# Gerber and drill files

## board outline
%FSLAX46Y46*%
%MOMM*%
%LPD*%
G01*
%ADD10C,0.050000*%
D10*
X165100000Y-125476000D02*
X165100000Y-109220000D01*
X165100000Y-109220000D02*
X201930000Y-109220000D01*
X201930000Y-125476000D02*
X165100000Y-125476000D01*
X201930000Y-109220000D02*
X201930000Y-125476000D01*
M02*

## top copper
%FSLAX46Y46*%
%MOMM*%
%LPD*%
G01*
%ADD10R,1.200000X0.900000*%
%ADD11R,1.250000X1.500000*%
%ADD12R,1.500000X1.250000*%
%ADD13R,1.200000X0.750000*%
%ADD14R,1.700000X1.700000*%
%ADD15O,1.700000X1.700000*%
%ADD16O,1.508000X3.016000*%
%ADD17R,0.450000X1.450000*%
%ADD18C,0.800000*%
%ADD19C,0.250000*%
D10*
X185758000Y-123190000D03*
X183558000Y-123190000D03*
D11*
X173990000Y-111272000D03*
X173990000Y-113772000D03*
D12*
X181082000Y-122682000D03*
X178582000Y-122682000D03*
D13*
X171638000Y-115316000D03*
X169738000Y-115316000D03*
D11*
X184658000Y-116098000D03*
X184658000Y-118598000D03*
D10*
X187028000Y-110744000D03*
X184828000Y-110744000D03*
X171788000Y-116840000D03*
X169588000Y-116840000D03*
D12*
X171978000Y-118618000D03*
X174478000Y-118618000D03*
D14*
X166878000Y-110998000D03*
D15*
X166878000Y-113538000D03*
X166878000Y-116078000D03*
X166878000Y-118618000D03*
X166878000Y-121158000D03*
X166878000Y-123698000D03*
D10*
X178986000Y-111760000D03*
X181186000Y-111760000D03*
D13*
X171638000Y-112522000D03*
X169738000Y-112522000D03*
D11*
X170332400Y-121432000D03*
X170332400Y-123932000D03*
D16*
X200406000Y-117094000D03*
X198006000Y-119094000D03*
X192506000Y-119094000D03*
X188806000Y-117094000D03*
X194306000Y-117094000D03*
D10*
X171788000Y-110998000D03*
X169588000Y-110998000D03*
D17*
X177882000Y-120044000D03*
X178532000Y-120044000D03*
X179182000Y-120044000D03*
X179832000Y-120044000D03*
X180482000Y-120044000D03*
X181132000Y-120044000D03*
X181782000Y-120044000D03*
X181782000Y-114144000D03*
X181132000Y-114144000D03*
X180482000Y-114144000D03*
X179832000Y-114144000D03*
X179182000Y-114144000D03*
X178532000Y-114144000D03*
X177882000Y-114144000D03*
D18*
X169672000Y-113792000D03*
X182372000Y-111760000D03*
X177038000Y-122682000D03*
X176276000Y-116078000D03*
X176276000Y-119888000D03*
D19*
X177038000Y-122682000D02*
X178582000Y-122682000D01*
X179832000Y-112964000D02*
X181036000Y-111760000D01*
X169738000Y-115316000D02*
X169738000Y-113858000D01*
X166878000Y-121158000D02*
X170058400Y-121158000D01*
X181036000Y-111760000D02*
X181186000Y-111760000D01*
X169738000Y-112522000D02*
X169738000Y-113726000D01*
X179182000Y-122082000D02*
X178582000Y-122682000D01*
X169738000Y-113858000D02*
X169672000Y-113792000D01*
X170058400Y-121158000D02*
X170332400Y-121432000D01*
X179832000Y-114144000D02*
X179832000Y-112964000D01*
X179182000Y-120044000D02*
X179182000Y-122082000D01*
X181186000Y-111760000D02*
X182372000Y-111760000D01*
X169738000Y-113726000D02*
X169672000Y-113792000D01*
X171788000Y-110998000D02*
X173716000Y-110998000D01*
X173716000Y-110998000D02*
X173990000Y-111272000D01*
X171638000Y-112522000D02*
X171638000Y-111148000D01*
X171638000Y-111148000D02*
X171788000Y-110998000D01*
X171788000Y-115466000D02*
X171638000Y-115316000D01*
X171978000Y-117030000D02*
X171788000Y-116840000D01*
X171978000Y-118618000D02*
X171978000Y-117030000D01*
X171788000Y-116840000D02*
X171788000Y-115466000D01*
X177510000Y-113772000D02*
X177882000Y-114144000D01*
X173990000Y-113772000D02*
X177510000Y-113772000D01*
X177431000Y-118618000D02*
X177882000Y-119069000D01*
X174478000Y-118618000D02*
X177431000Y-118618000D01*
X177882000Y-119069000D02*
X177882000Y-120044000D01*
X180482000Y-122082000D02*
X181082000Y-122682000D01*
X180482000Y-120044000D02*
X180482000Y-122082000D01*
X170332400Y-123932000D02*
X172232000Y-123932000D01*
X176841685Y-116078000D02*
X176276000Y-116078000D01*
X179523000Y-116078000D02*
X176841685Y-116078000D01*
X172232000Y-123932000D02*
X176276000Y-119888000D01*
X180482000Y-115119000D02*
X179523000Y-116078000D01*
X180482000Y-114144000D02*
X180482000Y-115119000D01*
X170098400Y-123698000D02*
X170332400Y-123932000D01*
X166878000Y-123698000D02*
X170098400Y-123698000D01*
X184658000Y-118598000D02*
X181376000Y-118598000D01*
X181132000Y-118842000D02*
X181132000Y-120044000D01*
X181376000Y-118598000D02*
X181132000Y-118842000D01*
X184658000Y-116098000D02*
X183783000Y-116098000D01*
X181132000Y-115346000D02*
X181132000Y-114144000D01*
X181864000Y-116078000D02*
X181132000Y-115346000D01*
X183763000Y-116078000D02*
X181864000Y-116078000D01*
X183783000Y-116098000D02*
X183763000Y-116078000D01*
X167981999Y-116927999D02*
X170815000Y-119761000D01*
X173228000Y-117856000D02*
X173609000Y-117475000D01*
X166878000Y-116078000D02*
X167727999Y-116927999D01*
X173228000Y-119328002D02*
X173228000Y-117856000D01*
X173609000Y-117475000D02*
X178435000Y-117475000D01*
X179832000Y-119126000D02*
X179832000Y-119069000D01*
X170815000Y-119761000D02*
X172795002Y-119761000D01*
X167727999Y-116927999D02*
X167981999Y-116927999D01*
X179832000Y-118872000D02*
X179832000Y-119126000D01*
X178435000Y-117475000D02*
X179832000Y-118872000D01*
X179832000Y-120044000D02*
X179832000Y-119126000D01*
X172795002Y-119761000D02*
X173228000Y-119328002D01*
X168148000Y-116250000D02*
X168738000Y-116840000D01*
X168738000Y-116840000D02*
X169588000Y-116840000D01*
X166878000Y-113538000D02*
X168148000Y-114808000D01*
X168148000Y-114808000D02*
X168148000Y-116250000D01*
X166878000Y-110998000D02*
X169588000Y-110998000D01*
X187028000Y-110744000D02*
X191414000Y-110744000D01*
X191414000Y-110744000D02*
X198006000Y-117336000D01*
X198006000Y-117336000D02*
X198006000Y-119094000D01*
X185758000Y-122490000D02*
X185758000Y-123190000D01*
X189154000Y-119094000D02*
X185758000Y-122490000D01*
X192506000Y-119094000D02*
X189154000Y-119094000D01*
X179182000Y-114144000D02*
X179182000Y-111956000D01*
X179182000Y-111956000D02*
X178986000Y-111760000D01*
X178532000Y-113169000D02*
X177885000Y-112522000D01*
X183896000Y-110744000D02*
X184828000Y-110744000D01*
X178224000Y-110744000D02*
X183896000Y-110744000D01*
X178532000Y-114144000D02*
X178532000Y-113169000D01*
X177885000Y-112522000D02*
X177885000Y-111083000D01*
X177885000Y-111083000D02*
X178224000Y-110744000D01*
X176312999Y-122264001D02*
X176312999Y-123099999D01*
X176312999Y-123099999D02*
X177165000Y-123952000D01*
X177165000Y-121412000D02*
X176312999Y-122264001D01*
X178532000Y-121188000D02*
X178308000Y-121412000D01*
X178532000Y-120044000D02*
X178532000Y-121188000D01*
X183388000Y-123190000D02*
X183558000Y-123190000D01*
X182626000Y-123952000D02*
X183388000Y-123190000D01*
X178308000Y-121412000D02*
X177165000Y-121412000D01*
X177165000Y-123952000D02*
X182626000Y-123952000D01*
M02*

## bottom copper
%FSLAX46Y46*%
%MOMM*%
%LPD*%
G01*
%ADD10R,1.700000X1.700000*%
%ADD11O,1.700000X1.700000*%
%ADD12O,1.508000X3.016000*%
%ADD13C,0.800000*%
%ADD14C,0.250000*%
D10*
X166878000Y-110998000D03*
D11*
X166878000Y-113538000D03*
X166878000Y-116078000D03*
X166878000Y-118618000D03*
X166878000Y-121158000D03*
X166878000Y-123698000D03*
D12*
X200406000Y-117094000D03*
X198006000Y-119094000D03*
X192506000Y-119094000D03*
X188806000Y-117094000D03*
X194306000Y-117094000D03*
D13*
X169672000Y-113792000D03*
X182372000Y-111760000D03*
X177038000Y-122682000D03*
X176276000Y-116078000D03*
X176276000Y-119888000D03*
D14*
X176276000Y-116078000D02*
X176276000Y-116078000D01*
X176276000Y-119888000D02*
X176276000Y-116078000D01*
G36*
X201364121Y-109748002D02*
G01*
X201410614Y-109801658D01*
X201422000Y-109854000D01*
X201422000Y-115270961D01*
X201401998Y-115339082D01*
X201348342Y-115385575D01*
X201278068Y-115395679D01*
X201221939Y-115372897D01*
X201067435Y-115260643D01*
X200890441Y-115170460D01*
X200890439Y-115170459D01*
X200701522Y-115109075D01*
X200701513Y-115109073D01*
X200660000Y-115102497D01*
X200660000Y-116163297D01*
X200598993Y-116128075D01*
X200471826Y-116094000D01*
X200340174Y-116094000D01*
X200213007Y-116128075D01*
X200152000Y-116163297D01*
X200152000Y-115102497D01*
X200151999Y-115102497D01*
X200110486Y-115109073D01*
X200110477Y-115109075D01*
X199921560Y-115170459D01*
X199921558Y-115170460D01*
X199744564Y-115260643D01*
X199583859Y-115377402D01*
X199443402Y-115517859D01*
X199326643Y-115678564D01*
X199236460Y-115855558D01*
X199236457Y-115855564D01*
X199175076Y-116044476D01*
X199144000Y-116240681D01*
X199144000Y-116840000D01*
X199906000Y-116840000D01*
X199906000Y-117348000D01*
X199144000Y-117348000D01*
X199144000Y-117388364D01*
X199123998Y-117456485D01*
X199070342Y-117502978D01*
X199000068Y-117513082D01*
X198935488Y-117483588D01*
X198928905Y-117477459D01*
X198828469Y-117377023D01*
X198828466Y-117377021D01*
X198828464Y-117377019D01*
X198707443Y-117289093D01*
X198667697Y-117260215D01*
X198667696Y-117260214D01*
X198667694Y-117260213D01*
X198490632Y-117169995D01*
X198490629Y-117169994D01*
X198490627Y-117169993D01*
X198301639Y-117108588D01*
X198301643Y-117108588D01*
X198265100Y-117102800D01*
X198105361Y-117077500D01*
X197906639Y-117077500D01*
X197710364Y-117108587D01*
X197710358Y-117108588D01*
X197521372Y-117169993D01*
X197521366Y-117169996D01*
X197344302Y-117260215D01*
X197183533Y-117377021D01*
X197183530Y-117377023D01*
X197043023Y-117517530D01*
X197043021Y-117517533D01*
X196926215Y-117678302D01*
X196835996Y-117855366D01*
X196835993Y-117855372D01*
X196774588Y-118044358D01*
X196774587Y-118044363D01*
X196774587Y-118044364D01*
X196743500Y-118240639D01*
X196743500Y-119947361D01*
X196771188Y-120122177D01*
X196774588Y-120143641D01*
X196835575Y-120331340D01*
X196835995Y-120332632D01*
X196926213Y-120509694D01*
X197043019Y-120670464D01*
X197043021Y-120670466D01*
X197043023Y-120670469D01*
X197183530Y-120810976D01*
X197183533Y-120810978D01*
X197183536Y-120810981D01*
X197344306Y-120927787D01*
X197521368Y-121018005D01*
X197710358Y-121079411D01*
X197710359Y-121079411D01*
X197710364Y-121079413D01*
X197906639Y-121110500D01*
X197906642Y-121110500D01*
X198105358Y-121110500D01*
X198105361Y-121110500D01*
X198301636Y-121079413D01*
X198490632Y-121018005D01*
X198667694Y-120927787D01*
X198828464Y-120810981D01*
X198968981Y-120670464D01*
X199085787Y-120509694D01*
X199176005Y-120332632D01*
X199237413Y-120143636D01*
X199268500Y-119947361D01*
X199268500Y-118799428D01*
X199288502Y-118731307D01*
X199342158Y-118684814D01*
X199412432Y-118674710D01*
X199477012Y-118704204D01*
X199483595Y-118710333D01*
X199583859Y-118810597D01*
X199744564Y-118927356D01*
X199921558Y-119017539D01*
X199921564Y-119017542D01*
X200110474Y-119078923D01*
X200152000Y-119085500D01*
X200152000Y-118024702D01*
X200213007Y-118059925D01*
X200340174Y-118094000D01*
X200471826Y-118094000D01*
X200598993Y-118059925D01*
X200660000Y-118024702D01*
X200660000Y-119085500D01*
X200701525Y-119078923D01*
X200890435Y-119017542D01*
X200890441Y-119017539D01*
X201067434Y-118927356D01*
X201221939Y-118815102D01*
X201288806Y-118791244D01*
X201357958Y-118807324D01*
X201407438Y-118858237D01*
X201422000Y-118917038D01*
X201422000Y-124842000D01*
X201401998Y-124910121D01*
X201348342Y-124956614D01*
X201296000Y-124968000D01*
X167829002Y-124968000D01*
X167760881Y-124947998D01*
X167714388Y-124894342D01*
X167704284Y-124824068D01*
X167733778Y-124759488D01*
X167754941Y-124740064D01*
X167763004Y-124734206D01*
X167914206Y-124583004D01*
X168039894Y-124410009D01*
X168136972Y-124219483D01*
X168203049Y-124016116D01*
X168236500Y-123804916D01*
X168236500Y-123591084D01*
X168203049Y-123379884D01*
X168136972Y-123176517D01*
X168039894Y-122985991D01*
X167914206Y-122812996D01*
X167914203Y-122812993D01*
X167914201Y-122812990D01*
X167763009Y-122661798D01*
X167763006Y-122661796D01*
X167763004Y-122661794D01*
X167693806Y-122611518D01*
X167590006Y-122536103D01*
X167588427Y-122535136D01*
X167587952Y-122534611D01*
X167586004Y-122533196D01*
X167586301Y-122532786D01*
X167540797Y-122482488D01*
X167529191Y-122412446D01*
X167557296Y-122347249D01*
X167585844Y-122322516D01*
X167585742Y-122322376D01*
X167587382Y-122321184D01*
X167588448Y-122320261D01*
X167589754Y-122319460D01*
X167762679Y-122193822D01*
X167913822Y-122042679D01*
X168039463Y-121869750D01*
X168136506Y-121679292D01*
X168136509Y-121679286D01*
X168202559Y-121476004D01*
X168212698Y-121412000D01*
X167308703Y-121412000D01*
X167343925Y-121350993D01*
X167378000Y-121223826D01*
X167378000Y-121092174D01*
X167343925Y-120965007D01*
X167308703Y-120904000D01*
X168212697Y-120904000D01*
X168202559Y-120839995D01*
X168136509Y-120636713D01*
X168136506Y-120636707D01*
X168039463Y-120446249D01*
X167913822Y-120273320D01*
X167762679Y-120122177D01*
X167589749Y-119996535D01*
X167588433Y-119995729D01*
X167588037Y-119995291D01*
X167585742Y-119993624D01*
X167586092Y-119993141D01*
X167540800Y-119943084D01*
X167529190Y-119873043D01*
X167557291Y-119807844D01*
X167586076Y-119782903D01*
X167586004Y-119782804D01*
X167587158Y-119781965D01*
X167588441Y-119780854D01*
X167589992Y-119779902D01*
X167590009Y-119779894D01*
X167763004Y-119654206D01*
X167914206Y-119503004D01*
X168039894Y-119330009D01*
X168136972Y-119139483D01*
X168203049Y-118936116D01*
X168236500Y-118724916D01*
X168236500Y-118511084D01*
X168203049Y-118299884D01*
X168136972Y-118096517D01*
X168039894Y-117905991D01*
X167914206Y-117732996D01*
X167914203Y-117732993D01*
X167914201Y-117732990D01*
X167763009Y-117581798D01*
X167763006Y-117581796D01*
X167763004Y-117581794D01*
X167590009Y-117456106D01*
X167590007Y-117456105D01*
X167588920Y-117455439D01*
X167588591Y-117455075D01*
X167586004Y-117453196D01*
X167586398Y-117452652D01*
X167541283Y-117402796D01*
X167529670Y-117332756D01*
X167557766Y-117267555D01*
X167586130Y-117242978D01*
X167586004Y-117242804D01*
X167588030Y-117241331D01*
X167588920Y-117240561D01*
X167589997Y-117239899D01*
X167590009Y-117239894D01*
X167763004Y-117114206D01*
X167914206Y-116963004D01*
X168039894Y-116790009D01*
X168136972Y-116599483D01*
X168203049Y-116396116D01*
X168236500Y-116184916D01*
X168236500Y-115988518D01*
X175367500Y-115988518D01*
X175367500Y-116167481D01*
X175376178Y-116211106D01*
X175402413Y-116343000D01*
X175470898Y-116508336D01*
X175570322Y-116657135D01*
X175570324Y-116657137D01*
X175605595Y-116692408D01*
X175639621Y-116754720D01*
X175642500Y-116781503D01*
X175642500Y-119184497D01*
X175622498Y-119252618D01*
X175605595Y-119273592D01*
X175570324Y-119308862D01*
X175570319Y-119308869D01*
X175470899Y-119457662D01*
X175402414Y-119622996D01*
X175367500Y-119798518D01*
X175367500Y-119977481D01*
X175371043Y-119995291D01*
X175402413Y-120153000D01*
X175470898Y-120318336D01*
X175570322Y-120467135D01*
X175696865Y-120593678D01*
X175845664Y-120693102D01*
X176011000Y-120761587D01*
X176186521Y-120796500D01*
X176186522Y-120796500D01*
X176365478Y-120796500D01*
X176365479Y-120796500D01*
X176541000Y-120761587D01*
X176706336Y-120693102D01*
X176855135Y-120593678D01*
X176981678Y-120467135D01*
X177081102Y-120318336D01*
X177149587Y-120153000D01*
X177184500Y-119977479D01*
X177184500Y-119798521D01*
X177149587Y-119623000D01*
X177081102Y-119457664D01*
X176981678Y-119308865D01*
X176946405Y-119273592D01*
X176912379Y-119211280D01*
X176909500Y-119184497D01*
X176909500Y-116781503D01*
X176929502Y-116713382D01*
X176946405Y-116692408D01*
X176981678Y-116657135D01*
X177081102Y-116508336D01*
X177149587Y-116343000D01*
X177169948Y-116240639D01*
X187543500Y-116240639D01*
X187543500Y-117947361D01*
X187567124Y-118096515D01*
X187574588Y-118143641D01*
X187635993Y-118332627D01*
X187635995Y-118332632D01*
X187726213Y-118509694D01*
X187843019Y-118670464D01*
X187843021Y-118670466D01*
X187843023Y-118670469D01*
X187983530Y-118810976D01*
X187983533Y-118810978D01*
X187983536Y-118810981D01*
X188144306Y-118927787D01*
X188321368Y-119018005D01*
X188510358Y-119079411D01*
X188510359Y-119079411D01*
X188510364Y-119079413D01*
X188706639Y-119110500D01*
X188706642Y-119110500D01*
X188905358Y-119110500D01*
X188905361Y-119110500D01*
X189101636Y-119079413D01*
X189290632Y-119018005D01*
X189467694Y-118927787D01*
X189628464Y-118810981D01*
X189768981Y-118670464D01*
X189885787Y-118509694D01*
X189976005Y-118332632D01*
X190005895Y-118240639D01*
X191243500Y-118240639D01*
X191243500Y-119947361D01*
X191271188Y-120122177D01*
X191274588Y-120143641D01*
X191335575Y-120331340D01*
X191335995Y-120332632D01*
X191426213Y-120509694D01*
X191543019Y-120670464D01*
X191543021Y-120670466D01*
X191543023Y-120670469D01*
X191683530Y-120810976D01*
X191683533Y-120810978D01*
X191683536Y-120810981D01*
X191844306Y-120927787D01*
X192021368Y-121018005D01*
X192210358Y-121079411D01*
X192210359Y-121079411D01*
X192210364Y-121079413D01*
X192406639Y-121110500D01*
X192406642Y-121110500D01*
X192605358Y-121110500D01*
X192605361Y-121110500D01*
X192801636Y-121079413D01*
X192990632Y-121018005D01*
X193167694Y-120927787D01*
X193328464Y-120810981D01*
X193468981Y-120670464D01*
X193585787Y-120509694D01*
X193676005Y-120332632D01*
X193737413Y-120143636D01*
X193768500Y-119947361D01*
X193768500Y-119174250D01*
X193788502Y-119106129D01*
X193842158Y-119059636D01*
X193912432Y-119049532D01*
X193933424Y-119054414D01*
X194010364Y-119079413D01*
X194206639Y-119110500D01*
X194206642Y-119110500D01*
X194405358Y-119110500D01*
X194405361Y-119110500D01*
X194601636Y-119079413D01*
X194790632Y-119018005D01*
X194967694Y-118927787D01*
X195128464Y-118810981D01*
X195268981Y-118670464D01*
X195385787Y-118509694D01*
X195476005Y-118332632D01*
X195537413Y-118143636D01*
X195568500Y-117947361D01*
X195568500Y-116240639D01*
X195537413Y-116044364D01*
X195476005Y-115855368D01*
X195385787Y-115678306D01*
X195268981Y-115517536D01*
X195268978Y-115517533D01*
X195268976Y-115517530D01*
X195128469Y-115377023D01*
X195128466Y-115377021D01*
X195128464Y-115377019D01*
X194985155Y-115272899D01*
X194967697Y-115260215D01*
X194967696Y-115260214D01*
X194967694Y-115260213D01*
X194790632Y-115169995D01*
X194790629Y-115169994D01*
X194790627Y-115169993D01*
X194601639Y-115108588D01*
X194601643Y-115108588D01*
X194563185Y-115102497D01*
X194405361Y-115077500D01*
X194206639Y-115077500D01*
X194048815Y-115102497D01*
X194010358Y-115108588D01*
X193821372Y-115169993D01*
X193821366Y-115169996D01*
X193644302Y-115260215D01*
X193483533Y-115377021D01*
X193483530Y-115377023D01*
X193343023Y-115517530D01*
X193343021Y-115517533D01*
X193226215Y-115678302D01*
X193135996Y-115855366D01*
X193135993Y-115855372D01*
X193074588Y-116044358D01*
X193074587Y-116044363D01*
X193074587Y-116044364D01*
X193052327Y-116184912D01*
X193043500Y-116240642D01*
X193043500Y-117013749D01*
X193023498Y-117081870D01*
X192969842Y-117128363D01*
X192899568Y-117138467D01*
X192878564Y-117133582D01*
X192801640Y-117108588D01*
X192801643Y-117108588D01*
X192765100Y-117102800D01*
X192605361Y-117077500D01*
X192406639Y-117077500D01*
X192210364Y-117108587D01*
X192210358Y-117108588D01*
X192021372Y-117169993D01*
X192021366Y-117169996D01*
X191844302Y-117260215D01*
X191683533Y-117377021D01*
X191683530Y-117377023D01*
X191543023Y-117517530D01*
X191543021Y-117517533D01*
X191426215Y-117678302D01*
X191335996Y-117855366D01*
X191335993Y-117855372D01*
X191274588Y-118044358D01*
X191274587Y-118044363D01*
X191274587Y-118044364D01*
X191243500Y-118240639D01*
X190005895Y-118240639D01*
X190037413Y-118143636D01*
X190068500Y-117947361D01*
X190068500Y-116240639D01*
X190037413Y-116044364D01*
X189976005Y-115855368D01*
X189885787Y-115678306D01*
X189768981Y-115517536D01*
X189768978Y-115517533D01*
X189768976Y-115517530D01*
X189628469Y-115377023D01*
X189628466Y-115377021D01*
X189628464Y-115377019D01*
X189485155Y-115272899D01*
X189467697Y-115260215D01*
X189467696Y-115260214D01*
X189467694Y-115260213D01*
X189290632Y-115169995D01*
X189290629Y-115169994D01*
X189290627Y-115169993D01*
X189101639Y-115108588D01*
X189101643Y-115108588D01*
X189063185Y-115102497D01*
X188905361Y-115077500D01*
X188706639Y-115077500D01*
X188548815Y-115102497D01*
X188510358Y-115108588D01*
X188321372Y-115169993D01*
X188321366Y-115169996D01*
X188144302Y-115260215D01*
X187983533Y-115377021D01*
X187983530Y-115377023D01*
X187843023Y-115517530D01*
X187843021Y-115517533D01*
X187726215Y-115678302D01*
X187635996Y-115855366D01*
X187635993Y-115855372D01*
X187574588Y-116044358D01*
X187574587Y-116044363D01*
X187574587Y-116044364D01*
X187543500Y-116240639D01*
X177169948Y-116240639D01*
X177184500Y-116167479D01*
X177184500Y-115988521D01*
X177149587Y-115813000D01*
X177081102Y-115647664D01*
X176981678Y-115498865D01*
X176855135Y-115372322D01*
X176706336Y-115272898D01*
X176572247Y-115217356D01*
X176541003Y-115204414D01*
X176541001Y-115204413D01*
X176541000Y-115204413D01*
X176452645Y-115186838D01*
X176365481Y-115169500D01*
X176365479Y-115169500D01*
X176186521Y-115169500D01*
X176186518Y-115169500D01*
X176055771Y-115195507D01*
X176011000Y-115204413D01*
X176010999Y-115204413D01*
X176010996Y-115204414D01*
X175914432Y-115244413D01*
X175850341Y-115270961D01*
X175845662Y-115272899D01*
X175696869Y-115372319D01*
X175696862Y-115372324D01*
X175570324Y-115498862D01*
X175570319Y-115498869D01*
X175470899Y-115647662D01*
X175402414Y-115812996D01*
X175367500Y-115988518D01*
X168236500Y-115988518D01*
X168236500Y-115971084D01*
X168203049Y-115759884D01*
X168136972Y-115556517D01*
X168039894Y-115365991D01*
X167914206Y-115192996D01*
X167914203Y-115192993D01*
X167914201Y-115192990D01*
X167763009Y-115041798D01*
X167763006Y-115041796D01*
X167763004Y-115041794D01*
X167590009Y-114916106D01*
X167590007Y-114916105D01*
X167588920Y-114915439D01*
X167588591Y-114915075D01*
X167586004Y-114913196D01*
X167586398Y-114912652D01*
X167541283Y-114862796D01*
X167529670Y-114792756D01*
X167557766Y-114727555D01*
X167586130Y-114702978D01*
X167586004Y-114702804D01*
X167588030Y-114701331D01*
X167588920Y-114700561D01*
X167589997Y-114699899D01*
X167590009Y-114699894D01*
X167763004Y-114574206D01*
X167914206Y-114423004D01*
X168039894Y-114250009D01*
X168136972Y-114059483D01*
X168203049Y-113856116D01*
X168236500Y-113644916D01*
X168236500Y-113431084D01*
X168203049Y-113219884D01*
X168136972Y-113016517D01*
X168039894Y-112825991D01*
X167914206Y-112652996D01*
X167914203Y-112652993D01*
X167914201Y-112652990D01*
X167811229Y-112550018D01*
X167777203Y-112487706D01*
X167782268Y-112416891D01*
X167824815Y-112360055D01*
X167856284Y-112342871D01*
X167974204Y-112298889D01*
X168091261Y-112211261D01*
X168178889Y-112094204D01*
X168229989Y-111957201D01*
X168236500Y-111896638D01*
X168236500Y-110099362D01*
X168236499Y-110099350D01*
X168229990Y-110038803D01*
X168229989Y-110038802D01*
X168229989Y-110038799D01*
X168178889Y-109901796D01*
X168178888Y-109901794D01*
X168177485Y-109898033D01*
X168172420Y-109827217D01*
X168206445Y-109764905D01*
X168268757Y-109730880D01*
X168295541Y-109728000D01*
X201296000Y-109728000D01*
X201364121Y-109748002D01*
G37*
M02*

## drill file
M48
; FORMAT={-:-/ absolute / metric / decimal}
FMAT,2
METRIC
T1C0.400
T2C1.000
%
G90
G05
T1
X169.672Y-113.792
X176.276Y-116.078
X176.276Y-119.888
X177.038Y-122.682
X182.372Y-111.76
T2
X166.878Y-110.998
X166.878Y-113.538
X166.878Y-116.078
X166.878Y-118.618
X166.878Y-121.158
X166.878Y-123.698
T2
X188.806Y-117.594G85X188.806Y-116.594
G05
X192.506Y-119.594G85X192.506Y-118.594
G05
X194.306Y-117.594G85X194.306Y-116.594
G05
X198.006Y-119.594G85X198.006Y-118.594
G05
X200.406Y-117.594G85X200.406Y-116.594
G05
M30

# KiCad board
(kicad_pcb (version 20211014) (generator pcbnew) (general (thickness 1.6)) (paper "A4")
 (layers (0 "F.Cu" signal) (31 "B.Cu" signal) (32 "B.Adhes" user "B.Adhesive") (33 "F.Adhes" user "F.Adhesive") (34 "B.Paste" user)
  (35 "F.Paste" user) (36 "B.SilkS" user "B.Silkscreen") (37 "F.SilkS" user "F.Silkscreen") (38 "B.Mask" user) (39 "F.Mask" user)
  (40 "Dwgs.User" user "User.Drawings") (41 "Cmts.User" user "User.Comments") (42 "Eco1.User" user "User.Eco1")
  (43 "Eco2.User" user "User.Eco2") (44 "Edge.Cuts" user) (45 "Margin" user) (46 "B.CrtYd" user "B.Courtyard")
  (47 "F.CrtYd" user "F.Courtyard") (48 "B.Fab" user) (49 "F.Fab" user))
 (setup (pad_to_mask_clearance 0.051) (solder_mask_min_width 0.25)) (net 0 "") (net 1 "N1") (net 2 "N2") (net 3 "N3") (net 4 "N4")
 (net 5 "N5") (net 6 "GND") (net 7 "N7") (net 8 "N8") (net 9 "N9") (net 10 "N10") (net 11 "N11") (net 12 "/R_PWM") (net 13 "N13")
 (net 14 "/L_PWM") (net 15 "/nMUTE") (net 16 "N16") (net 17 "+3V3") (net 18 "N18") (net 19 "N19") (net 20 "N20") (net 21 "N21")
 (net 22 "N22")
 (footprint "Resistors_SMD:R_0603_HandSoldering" (layer "F.Cu") (at 184.658 123.19 180)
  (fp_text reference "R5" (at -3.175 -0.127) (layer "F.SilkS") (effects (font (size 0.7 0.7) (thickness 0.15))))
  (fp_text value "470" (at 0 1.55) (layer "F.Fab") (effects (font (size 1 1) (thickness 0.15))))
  (pad "1" smd rect locked (at -1.1 0 180) (size 1.2 0.9) (layers "F.Cu" "F.Paste" "F.Mask") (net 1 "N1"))
  (pad "2" smd rect locked (at 1.1 0 180) (size 1.2 0.9) (layers "F.Cu" "F.Paste" "F.Mask") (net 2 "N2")))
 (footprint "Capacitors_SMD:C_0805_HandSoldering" (layer "F.Cu") (at 173.99 112.522 -90)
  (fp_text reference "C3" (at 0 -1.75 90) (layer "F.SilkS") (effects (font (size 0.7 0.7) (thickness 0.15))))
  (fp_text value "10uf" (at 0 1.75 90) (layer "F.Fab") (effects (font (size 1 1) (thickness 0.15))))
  (pad "1" smd rect locked (at -1.25 0 270) (size 1.5 1.25) (layers "F.Cu" "F.Paste" "F.Mask") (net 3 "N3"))
  (pad "2" smd rect locked (at 1.25 0 270) (size 1.5 1.25) (layers "F.Cu" "F.Paste" "F.Mask") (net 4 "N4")))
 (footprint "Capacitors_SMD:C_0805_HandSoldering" (layer "F.Cu") (at 179.832 122.682 180)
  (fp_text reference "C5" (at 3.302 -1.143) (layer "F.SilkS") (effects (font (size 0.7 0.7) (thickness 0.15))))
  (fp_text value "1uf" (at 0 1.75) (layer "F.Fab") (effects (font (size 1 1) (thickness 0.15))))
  (pad "1" smd rect locked (at -1.25 0 180) (size 1.5 1.25) (layers "F.Cu" "F.Paste" "F.Mask") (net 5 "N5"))
  (pad "2" smd rect locked (at 1.25 0 180) (size 1.5 1.25) (layers "F.Cu" "F.Paste" "F.Mask") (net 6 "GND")))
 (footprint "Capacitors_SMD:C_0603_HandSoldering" (layer "F.Cu") (at 170.688 115.316 180)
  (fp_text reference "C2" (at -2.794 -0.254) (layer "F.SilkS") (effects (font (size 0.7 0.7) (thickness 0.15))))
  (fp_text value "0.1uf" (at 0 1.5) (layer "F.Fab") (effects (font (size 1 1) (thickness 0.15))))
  (pad "1" smd rect locked (at -0.95 0 180) (size 1.2 0.75) (layers "F.Cu" "F.Paste" "F.Mask") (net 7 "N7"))
  (pad "2" smd rect locked (at 0.95 0 180) (size 1.2 0.75) (layers "F.Cu" "F.Paste" "F.Mask") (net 6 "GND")))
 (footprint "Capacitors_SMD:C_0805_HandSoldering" (layer "F.Cu") (at 184.658 117.348 -90)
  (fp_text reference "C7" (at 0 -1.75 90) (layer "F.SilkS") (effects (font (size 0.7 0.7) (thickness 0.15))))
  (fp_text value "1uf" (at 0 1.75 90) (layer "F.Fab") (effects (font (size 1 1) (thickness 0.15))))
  (pad "1" smd rect locked (at -1.25 0 270) (size 1.5 1.25) (layers "F.Cu" "F.Paste" "F.Mask") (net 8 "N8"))
  (pad "2" smd rect locked (at 1.25 0 270) (size 1.5 1.25) (layers "F.Cu" "F.Paste" "F.Mask") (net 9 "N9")))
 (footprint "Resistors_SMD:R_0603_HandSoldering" (layer "F.Cu") (at 185.928 110.744 180)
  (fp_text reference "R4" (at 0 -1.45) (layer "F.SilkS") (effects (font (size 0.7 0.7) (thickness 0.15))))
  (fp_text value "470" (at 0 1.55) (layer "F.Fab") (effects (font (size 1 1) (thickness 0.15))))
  (pad "1" smd rect locked (at -1.1 0 180) (size 1.2 0.9) (layers "F.Cu" "F.Paste" "F.Mask") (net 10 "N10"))
  (pad "2" smd rect locked (at 1.1 0 180) (size 1.2 0.9) (layers "F.Cu" "F.Paste" "F.Mask") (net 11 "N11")))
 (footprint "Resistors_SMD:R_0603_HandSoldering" (layer "F.Cu") (at 170.688 116.84 180)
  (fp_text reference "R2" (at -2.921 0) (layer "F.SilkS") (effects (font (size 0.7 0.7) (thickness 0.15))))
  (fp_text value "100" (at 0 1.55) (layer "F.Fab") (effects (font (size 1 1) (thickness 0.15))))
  (pad "1" smd rect locked (at -1.1 0 180) (size 1.2 0.9) (layers "F.Cu" "F.Paste" "F.Mask") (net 7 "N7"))
  (pad "2" smd rect locked (at 1.1 0 180) (size 1.2 0.9) (layers "F.Cu" "F.Paste" "F.Mask") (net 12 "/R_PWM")))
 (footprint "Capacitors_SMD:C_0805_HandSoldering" (layer "F.Cu") (at 173.228 118.618)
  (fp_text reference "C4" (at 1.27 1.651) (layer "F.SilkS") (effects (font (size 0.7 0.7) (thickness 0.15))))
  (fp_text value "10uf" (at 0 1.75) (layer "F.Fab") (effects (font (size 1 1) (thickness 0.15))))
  (pad "1" smd rect locked (at -1.25 0) (size 1.5 1.25) (layers "F.Cu" "F.Paste" "F.Mask") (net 7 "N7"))
  (pad "2" smd rect locked (at 1.25 0) (size 1.5 1.25) (layers "F.Cu" "F.Paste" "F.Mask") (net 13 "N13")))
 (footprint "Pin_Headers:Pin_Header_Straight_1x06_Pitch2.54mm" (layer "F.Cu") (at 166.878 110.998)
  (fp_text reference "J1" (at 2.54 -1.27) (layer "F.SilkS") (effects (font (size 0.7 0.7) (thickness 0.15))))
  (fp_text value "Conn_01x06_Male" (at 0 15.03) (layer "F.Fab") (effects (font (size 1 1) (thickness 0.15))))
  (pad "1" thru_hole rect locked (at 0 0) (size 1.7 1.7) (drill 1) (layers *.Cu *.Mask) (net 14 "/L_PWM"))
  (pad "2" thru_hole oval locked (at 0 2.54) (size 1.7 1.7) (drill 1) (layers *.Cu *.Mask) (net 12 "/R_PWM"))
  (pad "3" thru_hole oval locked (at 0 5.08) (size 1.7 1.7) (drill 1) (layers *.Cu *.Mask) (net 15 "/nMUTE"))
  (pad "4" thru_hole oval locked (at 0 7.62) (size 1.7 1.7) (drill 1) (layers *.Cu *.Mask) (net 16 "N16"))
  (pad "5" thru_hole oval locked (at 0 10.16) (size 1.7 1.7) (drill 1) (layers *.Cu *.Mask) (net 6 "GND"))
  (pad "6" thru_hole oval locked (at 0 12.7) (size 1.7 1.7) (drill 1) (layers *.Cu *.Mask) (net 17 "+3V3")))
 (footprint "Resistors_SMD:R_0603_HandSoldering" (layer "F.Cu") (at 180.086 111.76)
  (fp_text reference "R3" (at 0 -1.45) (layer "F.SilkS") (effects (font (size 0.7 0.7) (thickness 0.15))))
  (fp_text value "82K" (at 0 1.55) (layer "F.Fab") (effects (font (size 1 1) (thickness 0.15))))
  (pad "1" smd rect locked (at -1.1 0) (size 1.2 0.9) (layers "F.Cu" "F.Paste" "F.Mask") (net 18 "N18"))
  (pad "2" smd rect locked (at 1.1 0) (size 1.2 0.9) (layers "F.Cu" "F.Paste" "F.Mask") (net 6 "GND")))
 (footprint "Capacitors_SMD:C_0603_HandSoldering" (layer "F.Cu") (at 170.688 112.522 180)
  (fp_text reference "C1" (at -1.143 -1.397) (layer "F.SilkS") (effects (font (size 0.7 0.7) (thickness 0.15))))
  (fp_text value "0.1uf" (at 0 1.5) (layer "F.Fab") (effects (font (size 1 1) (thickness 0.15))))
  (pad "1" smd rect locked (at -0.95 0 180) (size 1.2 0.75) (layers "F.Cu" "F.Paste" "F.Mask") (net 3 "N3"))
  (pad "2" smd rect locked (at 0.95 0 180) (size 1.2 0.75) (layers "F.Cu" "F.Paste" "F.Mask") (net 6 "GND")))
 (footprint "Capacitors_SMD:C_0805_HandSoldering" (layer "F.Cu") (at 170.3324 122.682 -90)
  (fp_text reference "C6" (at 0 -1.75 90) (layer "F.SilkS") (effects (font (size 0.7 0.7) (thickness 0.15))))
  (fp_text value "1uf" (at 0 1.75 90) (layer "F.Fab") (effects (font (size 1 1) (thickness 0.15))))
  (pad "1" smd rect locked (at -1.25 0 270) (size 1.5 1.25) (layers "F.Cu" "F.Paste" "F.Mask") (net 6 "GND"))
  (pad "2" smd rect locked (at 1.25 0 270) (size 1.5 1.25) (layers "F.Cu" "F.Paste" "F.Mask") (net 17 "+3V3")))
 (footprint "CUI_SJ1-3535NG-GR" (layer "F.Cu") (at 200.406 117.094 180)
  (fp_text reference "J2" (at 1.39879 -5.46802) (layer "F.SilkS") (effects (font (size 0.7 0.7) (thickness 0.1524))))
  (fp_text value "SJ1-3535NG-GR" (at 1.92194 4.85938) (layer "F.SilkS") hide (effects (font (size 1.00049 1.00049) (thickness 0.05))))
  (pad "1" thru_hole oval locked (at 0 0 90) (size 3.016 1.508) (drill oval 2 1) (layers *.Cu *.Mask) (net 6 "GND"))
  (pad "2" thru_hole oval locked (at 2.4 -2 90) (size 3.016 1.508) (drill oval 2 1) (layers *.Cu *.Mask) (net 10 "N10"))
  (pad "3" thru_hole oval locked (at 7.9 -2 90) (size 3.016 1.508) (drill oval 2 1) (layers *.Cu *.Mask) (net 1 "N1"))
  (pad "4" thru_hole oval locked (at 11.6 0 90) (size 3.016 1.508) (drill oval 2 1) (layers *.Cu *.Mask) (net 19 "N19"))
  (pad "5" thru_hole oval locked (at 6.1 0 90) (size 3.016 1.508) (drill oval 2 1) (layers *.Cu *.Mask) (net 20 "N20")))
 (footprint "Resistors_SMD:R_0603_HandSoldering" (layer "F.Cu") (at 170.688 110.998 180)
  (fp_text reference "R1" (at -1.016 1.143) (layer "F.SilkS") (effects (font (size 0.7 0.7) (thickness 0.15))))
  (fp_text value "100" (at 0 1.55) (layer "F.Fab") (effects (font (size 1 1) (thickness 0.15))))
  (pad "1" smd rect locked (at -1.1 0 180) (size 1.2 0.9) (layers "F.Cu" "F.Paste" "F.Mask") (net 3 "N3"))
  (pad "2" smd rect locked (at 1.1 0 180) (size 1.2 0.9) (layers "F.Cu" "F.Paste" "F.Mask") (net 14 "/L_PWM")))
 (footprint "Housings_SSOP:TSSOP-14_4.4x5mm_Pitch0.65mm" (layer "F.Cu") (at 179.832 117.094 90)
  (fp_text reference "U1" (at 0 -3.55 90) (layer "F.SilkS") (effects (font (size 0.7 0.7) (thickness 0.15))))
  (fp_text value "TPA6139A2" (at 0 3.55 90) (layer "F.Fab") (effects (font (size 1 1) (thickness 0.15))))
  (pad "1" smd rect locked (at -2.95 -1.95 90) (size 1.45 0.45) (layers "F.Cu" "F.Paste" "F.Mask") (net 13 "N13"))
  (pad "2" smd rect locked (at -2.95 -1.3 90) (size 1.45 0.45) (layers "F.Cu" "F.Paste" "F.Mask") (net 2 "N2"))
  (pad "3" smd rect locked (at -2.95 -0.65 90) (size 1.45 0.45) (layers "F.Cu" "F.Paste" "F.Mask") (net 6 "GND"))
  (pad "4" smd rect locked (at -2.95 0 90) (size 1.45 0.45) (layers "F.Cu" "F.Paste" "F.Mask") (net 15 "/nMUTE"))
  (pad "5" smd rect locked (at -2.95 0.65 90) (size 1.45 0.45) (layers "F.Cu" "F.Paste" "F.Mask") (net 5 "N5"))
  (pad "6" smd rect locked (at -2.95 1.3 90) (size 1.45 0.45) (layers "F.Cu" "F.Paste" "F.Mask") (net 9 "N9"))
  (pad "7" smd rect locked (at -2.95 1.95 90) (size 1.45 0.45) (layers "F.Cu" "F.Paste" "F.Mask") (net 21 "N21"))
  (pad "8" smd rect locked (at 2.95 1.95 90) (size 1.45 0.45) (layers "F.Cu" "F.Paste" "F.Mask") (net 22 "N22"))
  (pad "9" smd rect locked (at 2.95 1.3 90) (size 1.45 0.45) (layers "F.Cu" "F.Paste" "F.Mask") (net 8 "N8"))
  (pad "10" smd rect locked (at 2.95 0.65 90) (size 1.45 0.45) (layers "F.Cu" "F.Paste" "F.Mask") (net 17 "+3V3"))
  (pad "11" smd rect locked (at 2.95 0 90) (size 1.45 0.45) (layers "F.Cu" "F.Paste" "F.Mask") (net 6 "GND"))
  (pad "12" smd rect locked (at 2.95 -0.65 90) (size 1.45 0.45) (layers "F.Cu" "F.Paste" "F.Mask") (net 18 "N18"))
  (pad "13" smd rect locked (at 2.95 -1.3 90) (size 1.45 0.45) (layers "F.Cu" "F.Paste" "F.Mask") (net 11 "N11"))
  (pad "14" smd rect locked (at 2.95 -1.95 90) (size 1.45 0.45) (layers "F.Cu" "F.Paste" "F.Mask") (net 4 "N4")))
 (gr_line (start 165.1 125.476) (end 165.1 109.22) (layer "Edge.Cuts") (width 0.05))
 (gr_line (start 165.1 109.22) (end 201.93 109.22) (layer "Edge.Cuts") (width 0.05))
 (gr_line (start 201.93 125.476) (end 165.1 125.476) (layer "Edge.Cuts") (width 0.05))
 (gr_line (start 201.93 109.22) (end 201.93 125.476) (layer "Edge.Cuts") (width 0.05))
 (segment (start 177.038 122.682) (end 178.582 122.682) (width 0.25) (layer "F.Cu") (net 6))
 (segment (start 179.832 112.964) (end 181.036 111.76) (width 0.25) (layer "F.Cu") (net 6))
 (segment (start 169.738 115.316) (end 169.738 113.858) (width 0.25) (layer "F.Cu") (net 6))
 (segment (start 166.878 121.158) (end 170.0584 121.158) (width 0.25) (layer "F.Cu") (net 6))
 (segment (start 181.036 111.76) (end 181.186 111.76) (width 0.25) (layer "F.Cu") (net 6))
 (segment (start 169.738 112.522) (end 169.738 113.726) (width 0.25) (layer "F.Cu") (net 6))
 (segment (start 179.182 122.082) (end 178.582 122.682) (width 0.25) (layer "F.Cu") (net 6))
 (segment (start 169.738 113.858) (end 169.672 113.792) (width 0.25) (layer "F.Cu") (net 6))
 (segment (start 170.0584 121.158) (end 170.3324 121.432) (width 0.25) (layer "F.Cu") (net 6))
 (segment (start 179.832 114.144) (end 179.832 112.964) (width 0.25) (layer "F.Cu") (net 6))
 (segment (start 179.182 120.044) (end 179.182 122.082) (width 0.25) (layer "F.Cu") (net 6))
 (segment (start 181.186 111.76) (end 182.372 111.76) (width 0.25) (layer "F.Cu") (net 6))
 (segment (start 169.738 113.726) (end 169.672 113.792) (width 0.25) (layer "F.Cu") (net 6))
 (via (at 169.672 113.792) (size 0.8) (drill 0.4) (layers "F.Cu" "B.Cu") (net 6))
 (via (at 182.372 111.76) (size 0.8) (drill 0.4) (layers "F.Cu" "B.Cu") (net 6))
 (via (at 177.038 122.682) (size 0.8) (drill 0.4) (layers "F.Cu" "B.Cu") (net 6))
 (segment (start 171.788 110.998) (end 173.716 110.998) (width 0.25) (layer "F.Cu") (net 3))
 (segment (start 173.716 110.998) (end 173.99 111.272) (width 0.25) (layer "F.Cu") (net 3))
 (segment (start 171.638 112.522) (end 171.638 111.148) (width 0.25) (layer "F.Cu") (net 3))
 (segment (start 171.638 111.148) (end 171.788 110.998) (width 0.25) (layer "F.Cu") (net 3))
 (segment (start 171.788 115.466) (end 171.638 115.316) (width 0.25) (layer "F.Cu") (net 7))
 (segment (start 171.978 117.03) (end 171.788 116.84) (width 0.25) (layer "F.Cu") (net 7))
 (segment (start 171.978 118.618) (end 171.978 117.03) (width 0.25) (layer "F.Cu") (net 7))
 (segment (start 171.788 116.84) (end 171.788 115.466) (width 0.25) (layer "F.Cu") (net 7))
 (segment (start 177.51 113.772) (end 177.882 114.144) (width 0.25) (layer "F.Cu") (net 4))
 (segment (start 173.99 113.772) (end 177.51 113.772) (width 0.25) (layer "F.Cu") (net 4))
 (segment (start 177.431 118.618) (end 177.882 119.069) (width 0.25) (layer "F.Cu") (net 13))
 (segment (start 174.478 118.618) (end 177.431 118.618) (width 0.25) (layer "F.Cu") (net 13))
 (segment (start 177.882 119.069) (end 177.882 120.044) (width 0.25) (layer "F.Cu") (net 13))
 (segment (start 180.482 122.082) (end 181.082 122.682) (width 0.25) (layer "F.Cu") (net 5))
 (segment (start 180.482 120.044) (end 180.482 122.082) (width 0.25) (layer "F.Cu") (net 5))
 (segment (start 170.3324 123.932) (end 172.232 123.932) (width 0.25) (layer "F.Cu") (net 17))
 (segment (start 176.841685 116.078) (end 176.276 116.078) (width 0.25) (layer "F.Cu") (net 17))
 (segment (start 179.523 116.078) (end 176.841685 116.078) (width 0.25) (layer "F.Cu") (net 17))
 (segment (start 172.232 123.932) (end 176.276 119.888) (width 0.25) (layer "F.Cu") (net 17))
 (segment (start 180.482 115.119) (end 179.523 116.078) (width 0.25) (layer "F.Cu") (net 17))
 (segment (start 180.482 114.144) (end 180.482 115.119) (width 0.25) (layer "F.Cu") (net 17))
 (segment (start 170.0984 123.698) (end 170.3324 123.932) (width 0.25) (layer "F.Cu") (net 17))
 (segment (start 166.878 123.698) (end 170.0984 123.698) (width 0.25) (layer "F.Cu") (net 17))
 (via (at 176.276 116.078) (size 0.8) (drill 0.4) (layers "F.Cu" "B.Cu") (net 17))
 (via (at 176.276 119.888) (size 0.8) (drill 0.4) (layers "F.Cu" "B.Cu") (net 17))
 (segment (start 176.276 116.078) (end 176.276 116.078) (width 0.25) (layer "B.Cu") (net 17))
 (segment (start 176.276 119.888) (end 176.276 116.078) (width 0.25) (layer "B.Cu") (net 17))
 (segment (start 184.658 118.598) (end 181.376 118.598) (width 0.25) (layer "F.Cu") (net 9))
 (segment (start 181.132 118.842) (end 181.132 120.044) (width 0.25) (layer "F.Cu") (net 9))
 (segment (start 181.376 118.598) (end 181.132 118.842) (width 0.25) (layer "F.Cu") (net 9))
 (segment (start 184.658 116.098) (end 183.783 116.098) (width 0.25) (layer "F.Cu") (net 8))
 (segment (start 181.132 115.346) (end 181.132 114.144) (width 0.25) (layer "F.Cu") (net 8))
 (segment (start 181.864 116.078) (end 181.132 115.346) (width 0.25) (layer "F.Cu") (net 8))
 (segment (start 183.763 116.078) (end 181.864 116.078) (width 0.25) (layer "F.Cu") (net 8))
 (segment (start 183.783 116.098) (end 183.763 116.078) (width 0.25) (layer "F.Cu") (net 8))
 (segment (start 167.981999 116.927999) (end 170.815 119.761) (width 0.25) (layer "F.Cu") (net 15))
 (segment (start 173.228 117.856) (end 173.609 117.475) (width 0.25) (layer "F.Cu") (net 15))
 (segment (start 166.878 116.078) (end 167.727999 116.927999) (width 0.25) (layer "F.Cu") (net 15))
 (segment (start 173.228 119.328002) (end 173.228 117.856) (width 0.25) (layer "F.Cu") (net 15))
 (segment (start 173.609 117.475) (end 178.435 117.475) (width 0.25) (layer "F.Cu") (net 15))
 (segment (start 179.832 119.126) (end 179.832 119.069) (width 0.25) (layer "F.Cu") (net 15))
 (segment (start 170.815 119.761) (end 172.795002 119.761) (width 0.25) (layer "F.Cu") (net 15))
 (segment (start 167.727999 116.927999) (end 167.981999 116.927999) (width 0.25) (layer "F.Cu") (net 15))
 (segment (start 179.832 118.872) (end 179.832 119.126) (width 0.25) (layer "F.Cu") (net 15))
 (segment (start 178.435 117.475) (end 179.832 118.872) (width 0.25) (layer "F.Cu") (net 15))
 (segment (start 179.832 120.044) (end 179.832 119.126) (width 0.25) (layer "F.Cu") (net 15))
 (segment (start 172.795002 119.761) (end 173.228 119.328002) (width 0.25) (layer "F.Cu") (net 15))
 (segment (start 168.148 116.25) (end 168.738 116.84) (width 0.25) (layer "F.Cu") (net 12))
 (segment (start 168.738 116.84) (end 169.588 116.84) (width 0.25) (layer "F.Cu") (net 12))
 (segment (start 166.878 113.538) (end 168.148 114.808) (width 0.25) (layer "F.Cu") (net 12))
 (segment (start 168.148 114.808) (end 168.148 116.25) (width 0.25) (layer "F.Cu") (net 12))
 (segment (start 166.878 110.998) (end 169.588 110.998) (width 0.25) (layer "F.Cu") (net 14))
 (segment (start 187.028 110.744) (end 191.414 110.744) (width 0.25) (layer "F.Cu") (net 10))
 (segment (start 191.414 110.744) (end 198.006 117.336) (width 0.25) (layer "F.Cu") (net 10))
 (segment (start 198.006 117.336) (end 198.006 119.094) (width 0.25) (layer "F.Cu") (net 10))
 (segment (start 185.758 122.49) (end 185.758 123.19) (width 0.25) (layer "F.Cu") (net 1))
 (segment (start 189.154 119.094) (end 185.758 122.49) (width 0.25) (layer "F.Cu") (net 1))
 (segment (start 192.506 119.094) (end 189.154 119.094) (width 0.25) (layer "F.Cu") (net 1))
 (segment (start 179.182 114.144) (end 179.182 111.956) (width 0.25) (layer "F.Cu") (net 18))
 (segment (start 179.182 111.956) (end 178.986 111.76) (width 0.25) (layer "F.Cu") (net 18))
 (segment (start 178.532 113.169) (end 177.885 112.522) (width 0.25) (layer "F.Cu") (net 11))
 (segment (start 183.896 110.744) (end 184.828 110.744) (width 0.25) (layer "F.Cu") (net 11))
 (segment (start 178.224 110.744) (end 183.896 110.744) (width 0.25) (layer "F.Cu") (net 11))
 (segment (start 178.532 114.144) (end 178.532 113.169) (width 0.25) (layer "F.Cu") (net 11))
 (segment (start 177.885 112.522) (end 177.885 111.083) (width 0.25) (layer "F.Cu") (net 11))
 (segment (start 177.885 111.083) (end 178.224 110.744) (width 0.25) (layer "F.Cu") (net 11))
 (segment (start 176.312999 122.264001) (end 176.312999 123.099999) (width 0.25) (layer "F.Cu") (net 2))
 (segment (start 176.312999 123.099999) (end 177.165 123.952) (width 0.25) (layer "F.Cu") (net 2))
 (segment (start 177.165 121.412) (end 176.312999 122.264001) (width 0.25) (layer "F.Cu") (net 2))
 (segment (start 178.532 121.188) (end 178.308 121.412) (width 0.25) (layer "F.Cu") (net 2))
 (segment (start 178.532 120.044) (end 178.532 121.188) (width 0.25) (layer "F.Cu") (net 2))
 (segment (start 183.388 123.19) (end 183.558 123.19) (width 0.25) (layer "F.Cu") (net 2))
 (segment (start 182.626 123.952) (end 183.388 123.19) (width 0.25) (layer "F.Cu") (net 2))
 (segment (start 178.308 121.412) (end 177.165 121.412) (width 0.25) (layer "F.Cu") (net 2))
 (segment (start 177.165 123.952) (end 182.626 123.952) (width 0.25) (layer "F.Cu") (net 2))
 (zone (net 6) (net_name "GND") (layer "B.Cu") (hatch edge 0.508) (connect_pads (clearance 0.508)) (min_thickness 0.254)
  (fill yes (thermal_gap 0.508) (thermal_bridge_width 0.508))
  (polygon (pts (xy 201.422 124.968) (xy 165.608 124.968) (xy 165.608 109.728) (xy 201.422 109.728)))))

